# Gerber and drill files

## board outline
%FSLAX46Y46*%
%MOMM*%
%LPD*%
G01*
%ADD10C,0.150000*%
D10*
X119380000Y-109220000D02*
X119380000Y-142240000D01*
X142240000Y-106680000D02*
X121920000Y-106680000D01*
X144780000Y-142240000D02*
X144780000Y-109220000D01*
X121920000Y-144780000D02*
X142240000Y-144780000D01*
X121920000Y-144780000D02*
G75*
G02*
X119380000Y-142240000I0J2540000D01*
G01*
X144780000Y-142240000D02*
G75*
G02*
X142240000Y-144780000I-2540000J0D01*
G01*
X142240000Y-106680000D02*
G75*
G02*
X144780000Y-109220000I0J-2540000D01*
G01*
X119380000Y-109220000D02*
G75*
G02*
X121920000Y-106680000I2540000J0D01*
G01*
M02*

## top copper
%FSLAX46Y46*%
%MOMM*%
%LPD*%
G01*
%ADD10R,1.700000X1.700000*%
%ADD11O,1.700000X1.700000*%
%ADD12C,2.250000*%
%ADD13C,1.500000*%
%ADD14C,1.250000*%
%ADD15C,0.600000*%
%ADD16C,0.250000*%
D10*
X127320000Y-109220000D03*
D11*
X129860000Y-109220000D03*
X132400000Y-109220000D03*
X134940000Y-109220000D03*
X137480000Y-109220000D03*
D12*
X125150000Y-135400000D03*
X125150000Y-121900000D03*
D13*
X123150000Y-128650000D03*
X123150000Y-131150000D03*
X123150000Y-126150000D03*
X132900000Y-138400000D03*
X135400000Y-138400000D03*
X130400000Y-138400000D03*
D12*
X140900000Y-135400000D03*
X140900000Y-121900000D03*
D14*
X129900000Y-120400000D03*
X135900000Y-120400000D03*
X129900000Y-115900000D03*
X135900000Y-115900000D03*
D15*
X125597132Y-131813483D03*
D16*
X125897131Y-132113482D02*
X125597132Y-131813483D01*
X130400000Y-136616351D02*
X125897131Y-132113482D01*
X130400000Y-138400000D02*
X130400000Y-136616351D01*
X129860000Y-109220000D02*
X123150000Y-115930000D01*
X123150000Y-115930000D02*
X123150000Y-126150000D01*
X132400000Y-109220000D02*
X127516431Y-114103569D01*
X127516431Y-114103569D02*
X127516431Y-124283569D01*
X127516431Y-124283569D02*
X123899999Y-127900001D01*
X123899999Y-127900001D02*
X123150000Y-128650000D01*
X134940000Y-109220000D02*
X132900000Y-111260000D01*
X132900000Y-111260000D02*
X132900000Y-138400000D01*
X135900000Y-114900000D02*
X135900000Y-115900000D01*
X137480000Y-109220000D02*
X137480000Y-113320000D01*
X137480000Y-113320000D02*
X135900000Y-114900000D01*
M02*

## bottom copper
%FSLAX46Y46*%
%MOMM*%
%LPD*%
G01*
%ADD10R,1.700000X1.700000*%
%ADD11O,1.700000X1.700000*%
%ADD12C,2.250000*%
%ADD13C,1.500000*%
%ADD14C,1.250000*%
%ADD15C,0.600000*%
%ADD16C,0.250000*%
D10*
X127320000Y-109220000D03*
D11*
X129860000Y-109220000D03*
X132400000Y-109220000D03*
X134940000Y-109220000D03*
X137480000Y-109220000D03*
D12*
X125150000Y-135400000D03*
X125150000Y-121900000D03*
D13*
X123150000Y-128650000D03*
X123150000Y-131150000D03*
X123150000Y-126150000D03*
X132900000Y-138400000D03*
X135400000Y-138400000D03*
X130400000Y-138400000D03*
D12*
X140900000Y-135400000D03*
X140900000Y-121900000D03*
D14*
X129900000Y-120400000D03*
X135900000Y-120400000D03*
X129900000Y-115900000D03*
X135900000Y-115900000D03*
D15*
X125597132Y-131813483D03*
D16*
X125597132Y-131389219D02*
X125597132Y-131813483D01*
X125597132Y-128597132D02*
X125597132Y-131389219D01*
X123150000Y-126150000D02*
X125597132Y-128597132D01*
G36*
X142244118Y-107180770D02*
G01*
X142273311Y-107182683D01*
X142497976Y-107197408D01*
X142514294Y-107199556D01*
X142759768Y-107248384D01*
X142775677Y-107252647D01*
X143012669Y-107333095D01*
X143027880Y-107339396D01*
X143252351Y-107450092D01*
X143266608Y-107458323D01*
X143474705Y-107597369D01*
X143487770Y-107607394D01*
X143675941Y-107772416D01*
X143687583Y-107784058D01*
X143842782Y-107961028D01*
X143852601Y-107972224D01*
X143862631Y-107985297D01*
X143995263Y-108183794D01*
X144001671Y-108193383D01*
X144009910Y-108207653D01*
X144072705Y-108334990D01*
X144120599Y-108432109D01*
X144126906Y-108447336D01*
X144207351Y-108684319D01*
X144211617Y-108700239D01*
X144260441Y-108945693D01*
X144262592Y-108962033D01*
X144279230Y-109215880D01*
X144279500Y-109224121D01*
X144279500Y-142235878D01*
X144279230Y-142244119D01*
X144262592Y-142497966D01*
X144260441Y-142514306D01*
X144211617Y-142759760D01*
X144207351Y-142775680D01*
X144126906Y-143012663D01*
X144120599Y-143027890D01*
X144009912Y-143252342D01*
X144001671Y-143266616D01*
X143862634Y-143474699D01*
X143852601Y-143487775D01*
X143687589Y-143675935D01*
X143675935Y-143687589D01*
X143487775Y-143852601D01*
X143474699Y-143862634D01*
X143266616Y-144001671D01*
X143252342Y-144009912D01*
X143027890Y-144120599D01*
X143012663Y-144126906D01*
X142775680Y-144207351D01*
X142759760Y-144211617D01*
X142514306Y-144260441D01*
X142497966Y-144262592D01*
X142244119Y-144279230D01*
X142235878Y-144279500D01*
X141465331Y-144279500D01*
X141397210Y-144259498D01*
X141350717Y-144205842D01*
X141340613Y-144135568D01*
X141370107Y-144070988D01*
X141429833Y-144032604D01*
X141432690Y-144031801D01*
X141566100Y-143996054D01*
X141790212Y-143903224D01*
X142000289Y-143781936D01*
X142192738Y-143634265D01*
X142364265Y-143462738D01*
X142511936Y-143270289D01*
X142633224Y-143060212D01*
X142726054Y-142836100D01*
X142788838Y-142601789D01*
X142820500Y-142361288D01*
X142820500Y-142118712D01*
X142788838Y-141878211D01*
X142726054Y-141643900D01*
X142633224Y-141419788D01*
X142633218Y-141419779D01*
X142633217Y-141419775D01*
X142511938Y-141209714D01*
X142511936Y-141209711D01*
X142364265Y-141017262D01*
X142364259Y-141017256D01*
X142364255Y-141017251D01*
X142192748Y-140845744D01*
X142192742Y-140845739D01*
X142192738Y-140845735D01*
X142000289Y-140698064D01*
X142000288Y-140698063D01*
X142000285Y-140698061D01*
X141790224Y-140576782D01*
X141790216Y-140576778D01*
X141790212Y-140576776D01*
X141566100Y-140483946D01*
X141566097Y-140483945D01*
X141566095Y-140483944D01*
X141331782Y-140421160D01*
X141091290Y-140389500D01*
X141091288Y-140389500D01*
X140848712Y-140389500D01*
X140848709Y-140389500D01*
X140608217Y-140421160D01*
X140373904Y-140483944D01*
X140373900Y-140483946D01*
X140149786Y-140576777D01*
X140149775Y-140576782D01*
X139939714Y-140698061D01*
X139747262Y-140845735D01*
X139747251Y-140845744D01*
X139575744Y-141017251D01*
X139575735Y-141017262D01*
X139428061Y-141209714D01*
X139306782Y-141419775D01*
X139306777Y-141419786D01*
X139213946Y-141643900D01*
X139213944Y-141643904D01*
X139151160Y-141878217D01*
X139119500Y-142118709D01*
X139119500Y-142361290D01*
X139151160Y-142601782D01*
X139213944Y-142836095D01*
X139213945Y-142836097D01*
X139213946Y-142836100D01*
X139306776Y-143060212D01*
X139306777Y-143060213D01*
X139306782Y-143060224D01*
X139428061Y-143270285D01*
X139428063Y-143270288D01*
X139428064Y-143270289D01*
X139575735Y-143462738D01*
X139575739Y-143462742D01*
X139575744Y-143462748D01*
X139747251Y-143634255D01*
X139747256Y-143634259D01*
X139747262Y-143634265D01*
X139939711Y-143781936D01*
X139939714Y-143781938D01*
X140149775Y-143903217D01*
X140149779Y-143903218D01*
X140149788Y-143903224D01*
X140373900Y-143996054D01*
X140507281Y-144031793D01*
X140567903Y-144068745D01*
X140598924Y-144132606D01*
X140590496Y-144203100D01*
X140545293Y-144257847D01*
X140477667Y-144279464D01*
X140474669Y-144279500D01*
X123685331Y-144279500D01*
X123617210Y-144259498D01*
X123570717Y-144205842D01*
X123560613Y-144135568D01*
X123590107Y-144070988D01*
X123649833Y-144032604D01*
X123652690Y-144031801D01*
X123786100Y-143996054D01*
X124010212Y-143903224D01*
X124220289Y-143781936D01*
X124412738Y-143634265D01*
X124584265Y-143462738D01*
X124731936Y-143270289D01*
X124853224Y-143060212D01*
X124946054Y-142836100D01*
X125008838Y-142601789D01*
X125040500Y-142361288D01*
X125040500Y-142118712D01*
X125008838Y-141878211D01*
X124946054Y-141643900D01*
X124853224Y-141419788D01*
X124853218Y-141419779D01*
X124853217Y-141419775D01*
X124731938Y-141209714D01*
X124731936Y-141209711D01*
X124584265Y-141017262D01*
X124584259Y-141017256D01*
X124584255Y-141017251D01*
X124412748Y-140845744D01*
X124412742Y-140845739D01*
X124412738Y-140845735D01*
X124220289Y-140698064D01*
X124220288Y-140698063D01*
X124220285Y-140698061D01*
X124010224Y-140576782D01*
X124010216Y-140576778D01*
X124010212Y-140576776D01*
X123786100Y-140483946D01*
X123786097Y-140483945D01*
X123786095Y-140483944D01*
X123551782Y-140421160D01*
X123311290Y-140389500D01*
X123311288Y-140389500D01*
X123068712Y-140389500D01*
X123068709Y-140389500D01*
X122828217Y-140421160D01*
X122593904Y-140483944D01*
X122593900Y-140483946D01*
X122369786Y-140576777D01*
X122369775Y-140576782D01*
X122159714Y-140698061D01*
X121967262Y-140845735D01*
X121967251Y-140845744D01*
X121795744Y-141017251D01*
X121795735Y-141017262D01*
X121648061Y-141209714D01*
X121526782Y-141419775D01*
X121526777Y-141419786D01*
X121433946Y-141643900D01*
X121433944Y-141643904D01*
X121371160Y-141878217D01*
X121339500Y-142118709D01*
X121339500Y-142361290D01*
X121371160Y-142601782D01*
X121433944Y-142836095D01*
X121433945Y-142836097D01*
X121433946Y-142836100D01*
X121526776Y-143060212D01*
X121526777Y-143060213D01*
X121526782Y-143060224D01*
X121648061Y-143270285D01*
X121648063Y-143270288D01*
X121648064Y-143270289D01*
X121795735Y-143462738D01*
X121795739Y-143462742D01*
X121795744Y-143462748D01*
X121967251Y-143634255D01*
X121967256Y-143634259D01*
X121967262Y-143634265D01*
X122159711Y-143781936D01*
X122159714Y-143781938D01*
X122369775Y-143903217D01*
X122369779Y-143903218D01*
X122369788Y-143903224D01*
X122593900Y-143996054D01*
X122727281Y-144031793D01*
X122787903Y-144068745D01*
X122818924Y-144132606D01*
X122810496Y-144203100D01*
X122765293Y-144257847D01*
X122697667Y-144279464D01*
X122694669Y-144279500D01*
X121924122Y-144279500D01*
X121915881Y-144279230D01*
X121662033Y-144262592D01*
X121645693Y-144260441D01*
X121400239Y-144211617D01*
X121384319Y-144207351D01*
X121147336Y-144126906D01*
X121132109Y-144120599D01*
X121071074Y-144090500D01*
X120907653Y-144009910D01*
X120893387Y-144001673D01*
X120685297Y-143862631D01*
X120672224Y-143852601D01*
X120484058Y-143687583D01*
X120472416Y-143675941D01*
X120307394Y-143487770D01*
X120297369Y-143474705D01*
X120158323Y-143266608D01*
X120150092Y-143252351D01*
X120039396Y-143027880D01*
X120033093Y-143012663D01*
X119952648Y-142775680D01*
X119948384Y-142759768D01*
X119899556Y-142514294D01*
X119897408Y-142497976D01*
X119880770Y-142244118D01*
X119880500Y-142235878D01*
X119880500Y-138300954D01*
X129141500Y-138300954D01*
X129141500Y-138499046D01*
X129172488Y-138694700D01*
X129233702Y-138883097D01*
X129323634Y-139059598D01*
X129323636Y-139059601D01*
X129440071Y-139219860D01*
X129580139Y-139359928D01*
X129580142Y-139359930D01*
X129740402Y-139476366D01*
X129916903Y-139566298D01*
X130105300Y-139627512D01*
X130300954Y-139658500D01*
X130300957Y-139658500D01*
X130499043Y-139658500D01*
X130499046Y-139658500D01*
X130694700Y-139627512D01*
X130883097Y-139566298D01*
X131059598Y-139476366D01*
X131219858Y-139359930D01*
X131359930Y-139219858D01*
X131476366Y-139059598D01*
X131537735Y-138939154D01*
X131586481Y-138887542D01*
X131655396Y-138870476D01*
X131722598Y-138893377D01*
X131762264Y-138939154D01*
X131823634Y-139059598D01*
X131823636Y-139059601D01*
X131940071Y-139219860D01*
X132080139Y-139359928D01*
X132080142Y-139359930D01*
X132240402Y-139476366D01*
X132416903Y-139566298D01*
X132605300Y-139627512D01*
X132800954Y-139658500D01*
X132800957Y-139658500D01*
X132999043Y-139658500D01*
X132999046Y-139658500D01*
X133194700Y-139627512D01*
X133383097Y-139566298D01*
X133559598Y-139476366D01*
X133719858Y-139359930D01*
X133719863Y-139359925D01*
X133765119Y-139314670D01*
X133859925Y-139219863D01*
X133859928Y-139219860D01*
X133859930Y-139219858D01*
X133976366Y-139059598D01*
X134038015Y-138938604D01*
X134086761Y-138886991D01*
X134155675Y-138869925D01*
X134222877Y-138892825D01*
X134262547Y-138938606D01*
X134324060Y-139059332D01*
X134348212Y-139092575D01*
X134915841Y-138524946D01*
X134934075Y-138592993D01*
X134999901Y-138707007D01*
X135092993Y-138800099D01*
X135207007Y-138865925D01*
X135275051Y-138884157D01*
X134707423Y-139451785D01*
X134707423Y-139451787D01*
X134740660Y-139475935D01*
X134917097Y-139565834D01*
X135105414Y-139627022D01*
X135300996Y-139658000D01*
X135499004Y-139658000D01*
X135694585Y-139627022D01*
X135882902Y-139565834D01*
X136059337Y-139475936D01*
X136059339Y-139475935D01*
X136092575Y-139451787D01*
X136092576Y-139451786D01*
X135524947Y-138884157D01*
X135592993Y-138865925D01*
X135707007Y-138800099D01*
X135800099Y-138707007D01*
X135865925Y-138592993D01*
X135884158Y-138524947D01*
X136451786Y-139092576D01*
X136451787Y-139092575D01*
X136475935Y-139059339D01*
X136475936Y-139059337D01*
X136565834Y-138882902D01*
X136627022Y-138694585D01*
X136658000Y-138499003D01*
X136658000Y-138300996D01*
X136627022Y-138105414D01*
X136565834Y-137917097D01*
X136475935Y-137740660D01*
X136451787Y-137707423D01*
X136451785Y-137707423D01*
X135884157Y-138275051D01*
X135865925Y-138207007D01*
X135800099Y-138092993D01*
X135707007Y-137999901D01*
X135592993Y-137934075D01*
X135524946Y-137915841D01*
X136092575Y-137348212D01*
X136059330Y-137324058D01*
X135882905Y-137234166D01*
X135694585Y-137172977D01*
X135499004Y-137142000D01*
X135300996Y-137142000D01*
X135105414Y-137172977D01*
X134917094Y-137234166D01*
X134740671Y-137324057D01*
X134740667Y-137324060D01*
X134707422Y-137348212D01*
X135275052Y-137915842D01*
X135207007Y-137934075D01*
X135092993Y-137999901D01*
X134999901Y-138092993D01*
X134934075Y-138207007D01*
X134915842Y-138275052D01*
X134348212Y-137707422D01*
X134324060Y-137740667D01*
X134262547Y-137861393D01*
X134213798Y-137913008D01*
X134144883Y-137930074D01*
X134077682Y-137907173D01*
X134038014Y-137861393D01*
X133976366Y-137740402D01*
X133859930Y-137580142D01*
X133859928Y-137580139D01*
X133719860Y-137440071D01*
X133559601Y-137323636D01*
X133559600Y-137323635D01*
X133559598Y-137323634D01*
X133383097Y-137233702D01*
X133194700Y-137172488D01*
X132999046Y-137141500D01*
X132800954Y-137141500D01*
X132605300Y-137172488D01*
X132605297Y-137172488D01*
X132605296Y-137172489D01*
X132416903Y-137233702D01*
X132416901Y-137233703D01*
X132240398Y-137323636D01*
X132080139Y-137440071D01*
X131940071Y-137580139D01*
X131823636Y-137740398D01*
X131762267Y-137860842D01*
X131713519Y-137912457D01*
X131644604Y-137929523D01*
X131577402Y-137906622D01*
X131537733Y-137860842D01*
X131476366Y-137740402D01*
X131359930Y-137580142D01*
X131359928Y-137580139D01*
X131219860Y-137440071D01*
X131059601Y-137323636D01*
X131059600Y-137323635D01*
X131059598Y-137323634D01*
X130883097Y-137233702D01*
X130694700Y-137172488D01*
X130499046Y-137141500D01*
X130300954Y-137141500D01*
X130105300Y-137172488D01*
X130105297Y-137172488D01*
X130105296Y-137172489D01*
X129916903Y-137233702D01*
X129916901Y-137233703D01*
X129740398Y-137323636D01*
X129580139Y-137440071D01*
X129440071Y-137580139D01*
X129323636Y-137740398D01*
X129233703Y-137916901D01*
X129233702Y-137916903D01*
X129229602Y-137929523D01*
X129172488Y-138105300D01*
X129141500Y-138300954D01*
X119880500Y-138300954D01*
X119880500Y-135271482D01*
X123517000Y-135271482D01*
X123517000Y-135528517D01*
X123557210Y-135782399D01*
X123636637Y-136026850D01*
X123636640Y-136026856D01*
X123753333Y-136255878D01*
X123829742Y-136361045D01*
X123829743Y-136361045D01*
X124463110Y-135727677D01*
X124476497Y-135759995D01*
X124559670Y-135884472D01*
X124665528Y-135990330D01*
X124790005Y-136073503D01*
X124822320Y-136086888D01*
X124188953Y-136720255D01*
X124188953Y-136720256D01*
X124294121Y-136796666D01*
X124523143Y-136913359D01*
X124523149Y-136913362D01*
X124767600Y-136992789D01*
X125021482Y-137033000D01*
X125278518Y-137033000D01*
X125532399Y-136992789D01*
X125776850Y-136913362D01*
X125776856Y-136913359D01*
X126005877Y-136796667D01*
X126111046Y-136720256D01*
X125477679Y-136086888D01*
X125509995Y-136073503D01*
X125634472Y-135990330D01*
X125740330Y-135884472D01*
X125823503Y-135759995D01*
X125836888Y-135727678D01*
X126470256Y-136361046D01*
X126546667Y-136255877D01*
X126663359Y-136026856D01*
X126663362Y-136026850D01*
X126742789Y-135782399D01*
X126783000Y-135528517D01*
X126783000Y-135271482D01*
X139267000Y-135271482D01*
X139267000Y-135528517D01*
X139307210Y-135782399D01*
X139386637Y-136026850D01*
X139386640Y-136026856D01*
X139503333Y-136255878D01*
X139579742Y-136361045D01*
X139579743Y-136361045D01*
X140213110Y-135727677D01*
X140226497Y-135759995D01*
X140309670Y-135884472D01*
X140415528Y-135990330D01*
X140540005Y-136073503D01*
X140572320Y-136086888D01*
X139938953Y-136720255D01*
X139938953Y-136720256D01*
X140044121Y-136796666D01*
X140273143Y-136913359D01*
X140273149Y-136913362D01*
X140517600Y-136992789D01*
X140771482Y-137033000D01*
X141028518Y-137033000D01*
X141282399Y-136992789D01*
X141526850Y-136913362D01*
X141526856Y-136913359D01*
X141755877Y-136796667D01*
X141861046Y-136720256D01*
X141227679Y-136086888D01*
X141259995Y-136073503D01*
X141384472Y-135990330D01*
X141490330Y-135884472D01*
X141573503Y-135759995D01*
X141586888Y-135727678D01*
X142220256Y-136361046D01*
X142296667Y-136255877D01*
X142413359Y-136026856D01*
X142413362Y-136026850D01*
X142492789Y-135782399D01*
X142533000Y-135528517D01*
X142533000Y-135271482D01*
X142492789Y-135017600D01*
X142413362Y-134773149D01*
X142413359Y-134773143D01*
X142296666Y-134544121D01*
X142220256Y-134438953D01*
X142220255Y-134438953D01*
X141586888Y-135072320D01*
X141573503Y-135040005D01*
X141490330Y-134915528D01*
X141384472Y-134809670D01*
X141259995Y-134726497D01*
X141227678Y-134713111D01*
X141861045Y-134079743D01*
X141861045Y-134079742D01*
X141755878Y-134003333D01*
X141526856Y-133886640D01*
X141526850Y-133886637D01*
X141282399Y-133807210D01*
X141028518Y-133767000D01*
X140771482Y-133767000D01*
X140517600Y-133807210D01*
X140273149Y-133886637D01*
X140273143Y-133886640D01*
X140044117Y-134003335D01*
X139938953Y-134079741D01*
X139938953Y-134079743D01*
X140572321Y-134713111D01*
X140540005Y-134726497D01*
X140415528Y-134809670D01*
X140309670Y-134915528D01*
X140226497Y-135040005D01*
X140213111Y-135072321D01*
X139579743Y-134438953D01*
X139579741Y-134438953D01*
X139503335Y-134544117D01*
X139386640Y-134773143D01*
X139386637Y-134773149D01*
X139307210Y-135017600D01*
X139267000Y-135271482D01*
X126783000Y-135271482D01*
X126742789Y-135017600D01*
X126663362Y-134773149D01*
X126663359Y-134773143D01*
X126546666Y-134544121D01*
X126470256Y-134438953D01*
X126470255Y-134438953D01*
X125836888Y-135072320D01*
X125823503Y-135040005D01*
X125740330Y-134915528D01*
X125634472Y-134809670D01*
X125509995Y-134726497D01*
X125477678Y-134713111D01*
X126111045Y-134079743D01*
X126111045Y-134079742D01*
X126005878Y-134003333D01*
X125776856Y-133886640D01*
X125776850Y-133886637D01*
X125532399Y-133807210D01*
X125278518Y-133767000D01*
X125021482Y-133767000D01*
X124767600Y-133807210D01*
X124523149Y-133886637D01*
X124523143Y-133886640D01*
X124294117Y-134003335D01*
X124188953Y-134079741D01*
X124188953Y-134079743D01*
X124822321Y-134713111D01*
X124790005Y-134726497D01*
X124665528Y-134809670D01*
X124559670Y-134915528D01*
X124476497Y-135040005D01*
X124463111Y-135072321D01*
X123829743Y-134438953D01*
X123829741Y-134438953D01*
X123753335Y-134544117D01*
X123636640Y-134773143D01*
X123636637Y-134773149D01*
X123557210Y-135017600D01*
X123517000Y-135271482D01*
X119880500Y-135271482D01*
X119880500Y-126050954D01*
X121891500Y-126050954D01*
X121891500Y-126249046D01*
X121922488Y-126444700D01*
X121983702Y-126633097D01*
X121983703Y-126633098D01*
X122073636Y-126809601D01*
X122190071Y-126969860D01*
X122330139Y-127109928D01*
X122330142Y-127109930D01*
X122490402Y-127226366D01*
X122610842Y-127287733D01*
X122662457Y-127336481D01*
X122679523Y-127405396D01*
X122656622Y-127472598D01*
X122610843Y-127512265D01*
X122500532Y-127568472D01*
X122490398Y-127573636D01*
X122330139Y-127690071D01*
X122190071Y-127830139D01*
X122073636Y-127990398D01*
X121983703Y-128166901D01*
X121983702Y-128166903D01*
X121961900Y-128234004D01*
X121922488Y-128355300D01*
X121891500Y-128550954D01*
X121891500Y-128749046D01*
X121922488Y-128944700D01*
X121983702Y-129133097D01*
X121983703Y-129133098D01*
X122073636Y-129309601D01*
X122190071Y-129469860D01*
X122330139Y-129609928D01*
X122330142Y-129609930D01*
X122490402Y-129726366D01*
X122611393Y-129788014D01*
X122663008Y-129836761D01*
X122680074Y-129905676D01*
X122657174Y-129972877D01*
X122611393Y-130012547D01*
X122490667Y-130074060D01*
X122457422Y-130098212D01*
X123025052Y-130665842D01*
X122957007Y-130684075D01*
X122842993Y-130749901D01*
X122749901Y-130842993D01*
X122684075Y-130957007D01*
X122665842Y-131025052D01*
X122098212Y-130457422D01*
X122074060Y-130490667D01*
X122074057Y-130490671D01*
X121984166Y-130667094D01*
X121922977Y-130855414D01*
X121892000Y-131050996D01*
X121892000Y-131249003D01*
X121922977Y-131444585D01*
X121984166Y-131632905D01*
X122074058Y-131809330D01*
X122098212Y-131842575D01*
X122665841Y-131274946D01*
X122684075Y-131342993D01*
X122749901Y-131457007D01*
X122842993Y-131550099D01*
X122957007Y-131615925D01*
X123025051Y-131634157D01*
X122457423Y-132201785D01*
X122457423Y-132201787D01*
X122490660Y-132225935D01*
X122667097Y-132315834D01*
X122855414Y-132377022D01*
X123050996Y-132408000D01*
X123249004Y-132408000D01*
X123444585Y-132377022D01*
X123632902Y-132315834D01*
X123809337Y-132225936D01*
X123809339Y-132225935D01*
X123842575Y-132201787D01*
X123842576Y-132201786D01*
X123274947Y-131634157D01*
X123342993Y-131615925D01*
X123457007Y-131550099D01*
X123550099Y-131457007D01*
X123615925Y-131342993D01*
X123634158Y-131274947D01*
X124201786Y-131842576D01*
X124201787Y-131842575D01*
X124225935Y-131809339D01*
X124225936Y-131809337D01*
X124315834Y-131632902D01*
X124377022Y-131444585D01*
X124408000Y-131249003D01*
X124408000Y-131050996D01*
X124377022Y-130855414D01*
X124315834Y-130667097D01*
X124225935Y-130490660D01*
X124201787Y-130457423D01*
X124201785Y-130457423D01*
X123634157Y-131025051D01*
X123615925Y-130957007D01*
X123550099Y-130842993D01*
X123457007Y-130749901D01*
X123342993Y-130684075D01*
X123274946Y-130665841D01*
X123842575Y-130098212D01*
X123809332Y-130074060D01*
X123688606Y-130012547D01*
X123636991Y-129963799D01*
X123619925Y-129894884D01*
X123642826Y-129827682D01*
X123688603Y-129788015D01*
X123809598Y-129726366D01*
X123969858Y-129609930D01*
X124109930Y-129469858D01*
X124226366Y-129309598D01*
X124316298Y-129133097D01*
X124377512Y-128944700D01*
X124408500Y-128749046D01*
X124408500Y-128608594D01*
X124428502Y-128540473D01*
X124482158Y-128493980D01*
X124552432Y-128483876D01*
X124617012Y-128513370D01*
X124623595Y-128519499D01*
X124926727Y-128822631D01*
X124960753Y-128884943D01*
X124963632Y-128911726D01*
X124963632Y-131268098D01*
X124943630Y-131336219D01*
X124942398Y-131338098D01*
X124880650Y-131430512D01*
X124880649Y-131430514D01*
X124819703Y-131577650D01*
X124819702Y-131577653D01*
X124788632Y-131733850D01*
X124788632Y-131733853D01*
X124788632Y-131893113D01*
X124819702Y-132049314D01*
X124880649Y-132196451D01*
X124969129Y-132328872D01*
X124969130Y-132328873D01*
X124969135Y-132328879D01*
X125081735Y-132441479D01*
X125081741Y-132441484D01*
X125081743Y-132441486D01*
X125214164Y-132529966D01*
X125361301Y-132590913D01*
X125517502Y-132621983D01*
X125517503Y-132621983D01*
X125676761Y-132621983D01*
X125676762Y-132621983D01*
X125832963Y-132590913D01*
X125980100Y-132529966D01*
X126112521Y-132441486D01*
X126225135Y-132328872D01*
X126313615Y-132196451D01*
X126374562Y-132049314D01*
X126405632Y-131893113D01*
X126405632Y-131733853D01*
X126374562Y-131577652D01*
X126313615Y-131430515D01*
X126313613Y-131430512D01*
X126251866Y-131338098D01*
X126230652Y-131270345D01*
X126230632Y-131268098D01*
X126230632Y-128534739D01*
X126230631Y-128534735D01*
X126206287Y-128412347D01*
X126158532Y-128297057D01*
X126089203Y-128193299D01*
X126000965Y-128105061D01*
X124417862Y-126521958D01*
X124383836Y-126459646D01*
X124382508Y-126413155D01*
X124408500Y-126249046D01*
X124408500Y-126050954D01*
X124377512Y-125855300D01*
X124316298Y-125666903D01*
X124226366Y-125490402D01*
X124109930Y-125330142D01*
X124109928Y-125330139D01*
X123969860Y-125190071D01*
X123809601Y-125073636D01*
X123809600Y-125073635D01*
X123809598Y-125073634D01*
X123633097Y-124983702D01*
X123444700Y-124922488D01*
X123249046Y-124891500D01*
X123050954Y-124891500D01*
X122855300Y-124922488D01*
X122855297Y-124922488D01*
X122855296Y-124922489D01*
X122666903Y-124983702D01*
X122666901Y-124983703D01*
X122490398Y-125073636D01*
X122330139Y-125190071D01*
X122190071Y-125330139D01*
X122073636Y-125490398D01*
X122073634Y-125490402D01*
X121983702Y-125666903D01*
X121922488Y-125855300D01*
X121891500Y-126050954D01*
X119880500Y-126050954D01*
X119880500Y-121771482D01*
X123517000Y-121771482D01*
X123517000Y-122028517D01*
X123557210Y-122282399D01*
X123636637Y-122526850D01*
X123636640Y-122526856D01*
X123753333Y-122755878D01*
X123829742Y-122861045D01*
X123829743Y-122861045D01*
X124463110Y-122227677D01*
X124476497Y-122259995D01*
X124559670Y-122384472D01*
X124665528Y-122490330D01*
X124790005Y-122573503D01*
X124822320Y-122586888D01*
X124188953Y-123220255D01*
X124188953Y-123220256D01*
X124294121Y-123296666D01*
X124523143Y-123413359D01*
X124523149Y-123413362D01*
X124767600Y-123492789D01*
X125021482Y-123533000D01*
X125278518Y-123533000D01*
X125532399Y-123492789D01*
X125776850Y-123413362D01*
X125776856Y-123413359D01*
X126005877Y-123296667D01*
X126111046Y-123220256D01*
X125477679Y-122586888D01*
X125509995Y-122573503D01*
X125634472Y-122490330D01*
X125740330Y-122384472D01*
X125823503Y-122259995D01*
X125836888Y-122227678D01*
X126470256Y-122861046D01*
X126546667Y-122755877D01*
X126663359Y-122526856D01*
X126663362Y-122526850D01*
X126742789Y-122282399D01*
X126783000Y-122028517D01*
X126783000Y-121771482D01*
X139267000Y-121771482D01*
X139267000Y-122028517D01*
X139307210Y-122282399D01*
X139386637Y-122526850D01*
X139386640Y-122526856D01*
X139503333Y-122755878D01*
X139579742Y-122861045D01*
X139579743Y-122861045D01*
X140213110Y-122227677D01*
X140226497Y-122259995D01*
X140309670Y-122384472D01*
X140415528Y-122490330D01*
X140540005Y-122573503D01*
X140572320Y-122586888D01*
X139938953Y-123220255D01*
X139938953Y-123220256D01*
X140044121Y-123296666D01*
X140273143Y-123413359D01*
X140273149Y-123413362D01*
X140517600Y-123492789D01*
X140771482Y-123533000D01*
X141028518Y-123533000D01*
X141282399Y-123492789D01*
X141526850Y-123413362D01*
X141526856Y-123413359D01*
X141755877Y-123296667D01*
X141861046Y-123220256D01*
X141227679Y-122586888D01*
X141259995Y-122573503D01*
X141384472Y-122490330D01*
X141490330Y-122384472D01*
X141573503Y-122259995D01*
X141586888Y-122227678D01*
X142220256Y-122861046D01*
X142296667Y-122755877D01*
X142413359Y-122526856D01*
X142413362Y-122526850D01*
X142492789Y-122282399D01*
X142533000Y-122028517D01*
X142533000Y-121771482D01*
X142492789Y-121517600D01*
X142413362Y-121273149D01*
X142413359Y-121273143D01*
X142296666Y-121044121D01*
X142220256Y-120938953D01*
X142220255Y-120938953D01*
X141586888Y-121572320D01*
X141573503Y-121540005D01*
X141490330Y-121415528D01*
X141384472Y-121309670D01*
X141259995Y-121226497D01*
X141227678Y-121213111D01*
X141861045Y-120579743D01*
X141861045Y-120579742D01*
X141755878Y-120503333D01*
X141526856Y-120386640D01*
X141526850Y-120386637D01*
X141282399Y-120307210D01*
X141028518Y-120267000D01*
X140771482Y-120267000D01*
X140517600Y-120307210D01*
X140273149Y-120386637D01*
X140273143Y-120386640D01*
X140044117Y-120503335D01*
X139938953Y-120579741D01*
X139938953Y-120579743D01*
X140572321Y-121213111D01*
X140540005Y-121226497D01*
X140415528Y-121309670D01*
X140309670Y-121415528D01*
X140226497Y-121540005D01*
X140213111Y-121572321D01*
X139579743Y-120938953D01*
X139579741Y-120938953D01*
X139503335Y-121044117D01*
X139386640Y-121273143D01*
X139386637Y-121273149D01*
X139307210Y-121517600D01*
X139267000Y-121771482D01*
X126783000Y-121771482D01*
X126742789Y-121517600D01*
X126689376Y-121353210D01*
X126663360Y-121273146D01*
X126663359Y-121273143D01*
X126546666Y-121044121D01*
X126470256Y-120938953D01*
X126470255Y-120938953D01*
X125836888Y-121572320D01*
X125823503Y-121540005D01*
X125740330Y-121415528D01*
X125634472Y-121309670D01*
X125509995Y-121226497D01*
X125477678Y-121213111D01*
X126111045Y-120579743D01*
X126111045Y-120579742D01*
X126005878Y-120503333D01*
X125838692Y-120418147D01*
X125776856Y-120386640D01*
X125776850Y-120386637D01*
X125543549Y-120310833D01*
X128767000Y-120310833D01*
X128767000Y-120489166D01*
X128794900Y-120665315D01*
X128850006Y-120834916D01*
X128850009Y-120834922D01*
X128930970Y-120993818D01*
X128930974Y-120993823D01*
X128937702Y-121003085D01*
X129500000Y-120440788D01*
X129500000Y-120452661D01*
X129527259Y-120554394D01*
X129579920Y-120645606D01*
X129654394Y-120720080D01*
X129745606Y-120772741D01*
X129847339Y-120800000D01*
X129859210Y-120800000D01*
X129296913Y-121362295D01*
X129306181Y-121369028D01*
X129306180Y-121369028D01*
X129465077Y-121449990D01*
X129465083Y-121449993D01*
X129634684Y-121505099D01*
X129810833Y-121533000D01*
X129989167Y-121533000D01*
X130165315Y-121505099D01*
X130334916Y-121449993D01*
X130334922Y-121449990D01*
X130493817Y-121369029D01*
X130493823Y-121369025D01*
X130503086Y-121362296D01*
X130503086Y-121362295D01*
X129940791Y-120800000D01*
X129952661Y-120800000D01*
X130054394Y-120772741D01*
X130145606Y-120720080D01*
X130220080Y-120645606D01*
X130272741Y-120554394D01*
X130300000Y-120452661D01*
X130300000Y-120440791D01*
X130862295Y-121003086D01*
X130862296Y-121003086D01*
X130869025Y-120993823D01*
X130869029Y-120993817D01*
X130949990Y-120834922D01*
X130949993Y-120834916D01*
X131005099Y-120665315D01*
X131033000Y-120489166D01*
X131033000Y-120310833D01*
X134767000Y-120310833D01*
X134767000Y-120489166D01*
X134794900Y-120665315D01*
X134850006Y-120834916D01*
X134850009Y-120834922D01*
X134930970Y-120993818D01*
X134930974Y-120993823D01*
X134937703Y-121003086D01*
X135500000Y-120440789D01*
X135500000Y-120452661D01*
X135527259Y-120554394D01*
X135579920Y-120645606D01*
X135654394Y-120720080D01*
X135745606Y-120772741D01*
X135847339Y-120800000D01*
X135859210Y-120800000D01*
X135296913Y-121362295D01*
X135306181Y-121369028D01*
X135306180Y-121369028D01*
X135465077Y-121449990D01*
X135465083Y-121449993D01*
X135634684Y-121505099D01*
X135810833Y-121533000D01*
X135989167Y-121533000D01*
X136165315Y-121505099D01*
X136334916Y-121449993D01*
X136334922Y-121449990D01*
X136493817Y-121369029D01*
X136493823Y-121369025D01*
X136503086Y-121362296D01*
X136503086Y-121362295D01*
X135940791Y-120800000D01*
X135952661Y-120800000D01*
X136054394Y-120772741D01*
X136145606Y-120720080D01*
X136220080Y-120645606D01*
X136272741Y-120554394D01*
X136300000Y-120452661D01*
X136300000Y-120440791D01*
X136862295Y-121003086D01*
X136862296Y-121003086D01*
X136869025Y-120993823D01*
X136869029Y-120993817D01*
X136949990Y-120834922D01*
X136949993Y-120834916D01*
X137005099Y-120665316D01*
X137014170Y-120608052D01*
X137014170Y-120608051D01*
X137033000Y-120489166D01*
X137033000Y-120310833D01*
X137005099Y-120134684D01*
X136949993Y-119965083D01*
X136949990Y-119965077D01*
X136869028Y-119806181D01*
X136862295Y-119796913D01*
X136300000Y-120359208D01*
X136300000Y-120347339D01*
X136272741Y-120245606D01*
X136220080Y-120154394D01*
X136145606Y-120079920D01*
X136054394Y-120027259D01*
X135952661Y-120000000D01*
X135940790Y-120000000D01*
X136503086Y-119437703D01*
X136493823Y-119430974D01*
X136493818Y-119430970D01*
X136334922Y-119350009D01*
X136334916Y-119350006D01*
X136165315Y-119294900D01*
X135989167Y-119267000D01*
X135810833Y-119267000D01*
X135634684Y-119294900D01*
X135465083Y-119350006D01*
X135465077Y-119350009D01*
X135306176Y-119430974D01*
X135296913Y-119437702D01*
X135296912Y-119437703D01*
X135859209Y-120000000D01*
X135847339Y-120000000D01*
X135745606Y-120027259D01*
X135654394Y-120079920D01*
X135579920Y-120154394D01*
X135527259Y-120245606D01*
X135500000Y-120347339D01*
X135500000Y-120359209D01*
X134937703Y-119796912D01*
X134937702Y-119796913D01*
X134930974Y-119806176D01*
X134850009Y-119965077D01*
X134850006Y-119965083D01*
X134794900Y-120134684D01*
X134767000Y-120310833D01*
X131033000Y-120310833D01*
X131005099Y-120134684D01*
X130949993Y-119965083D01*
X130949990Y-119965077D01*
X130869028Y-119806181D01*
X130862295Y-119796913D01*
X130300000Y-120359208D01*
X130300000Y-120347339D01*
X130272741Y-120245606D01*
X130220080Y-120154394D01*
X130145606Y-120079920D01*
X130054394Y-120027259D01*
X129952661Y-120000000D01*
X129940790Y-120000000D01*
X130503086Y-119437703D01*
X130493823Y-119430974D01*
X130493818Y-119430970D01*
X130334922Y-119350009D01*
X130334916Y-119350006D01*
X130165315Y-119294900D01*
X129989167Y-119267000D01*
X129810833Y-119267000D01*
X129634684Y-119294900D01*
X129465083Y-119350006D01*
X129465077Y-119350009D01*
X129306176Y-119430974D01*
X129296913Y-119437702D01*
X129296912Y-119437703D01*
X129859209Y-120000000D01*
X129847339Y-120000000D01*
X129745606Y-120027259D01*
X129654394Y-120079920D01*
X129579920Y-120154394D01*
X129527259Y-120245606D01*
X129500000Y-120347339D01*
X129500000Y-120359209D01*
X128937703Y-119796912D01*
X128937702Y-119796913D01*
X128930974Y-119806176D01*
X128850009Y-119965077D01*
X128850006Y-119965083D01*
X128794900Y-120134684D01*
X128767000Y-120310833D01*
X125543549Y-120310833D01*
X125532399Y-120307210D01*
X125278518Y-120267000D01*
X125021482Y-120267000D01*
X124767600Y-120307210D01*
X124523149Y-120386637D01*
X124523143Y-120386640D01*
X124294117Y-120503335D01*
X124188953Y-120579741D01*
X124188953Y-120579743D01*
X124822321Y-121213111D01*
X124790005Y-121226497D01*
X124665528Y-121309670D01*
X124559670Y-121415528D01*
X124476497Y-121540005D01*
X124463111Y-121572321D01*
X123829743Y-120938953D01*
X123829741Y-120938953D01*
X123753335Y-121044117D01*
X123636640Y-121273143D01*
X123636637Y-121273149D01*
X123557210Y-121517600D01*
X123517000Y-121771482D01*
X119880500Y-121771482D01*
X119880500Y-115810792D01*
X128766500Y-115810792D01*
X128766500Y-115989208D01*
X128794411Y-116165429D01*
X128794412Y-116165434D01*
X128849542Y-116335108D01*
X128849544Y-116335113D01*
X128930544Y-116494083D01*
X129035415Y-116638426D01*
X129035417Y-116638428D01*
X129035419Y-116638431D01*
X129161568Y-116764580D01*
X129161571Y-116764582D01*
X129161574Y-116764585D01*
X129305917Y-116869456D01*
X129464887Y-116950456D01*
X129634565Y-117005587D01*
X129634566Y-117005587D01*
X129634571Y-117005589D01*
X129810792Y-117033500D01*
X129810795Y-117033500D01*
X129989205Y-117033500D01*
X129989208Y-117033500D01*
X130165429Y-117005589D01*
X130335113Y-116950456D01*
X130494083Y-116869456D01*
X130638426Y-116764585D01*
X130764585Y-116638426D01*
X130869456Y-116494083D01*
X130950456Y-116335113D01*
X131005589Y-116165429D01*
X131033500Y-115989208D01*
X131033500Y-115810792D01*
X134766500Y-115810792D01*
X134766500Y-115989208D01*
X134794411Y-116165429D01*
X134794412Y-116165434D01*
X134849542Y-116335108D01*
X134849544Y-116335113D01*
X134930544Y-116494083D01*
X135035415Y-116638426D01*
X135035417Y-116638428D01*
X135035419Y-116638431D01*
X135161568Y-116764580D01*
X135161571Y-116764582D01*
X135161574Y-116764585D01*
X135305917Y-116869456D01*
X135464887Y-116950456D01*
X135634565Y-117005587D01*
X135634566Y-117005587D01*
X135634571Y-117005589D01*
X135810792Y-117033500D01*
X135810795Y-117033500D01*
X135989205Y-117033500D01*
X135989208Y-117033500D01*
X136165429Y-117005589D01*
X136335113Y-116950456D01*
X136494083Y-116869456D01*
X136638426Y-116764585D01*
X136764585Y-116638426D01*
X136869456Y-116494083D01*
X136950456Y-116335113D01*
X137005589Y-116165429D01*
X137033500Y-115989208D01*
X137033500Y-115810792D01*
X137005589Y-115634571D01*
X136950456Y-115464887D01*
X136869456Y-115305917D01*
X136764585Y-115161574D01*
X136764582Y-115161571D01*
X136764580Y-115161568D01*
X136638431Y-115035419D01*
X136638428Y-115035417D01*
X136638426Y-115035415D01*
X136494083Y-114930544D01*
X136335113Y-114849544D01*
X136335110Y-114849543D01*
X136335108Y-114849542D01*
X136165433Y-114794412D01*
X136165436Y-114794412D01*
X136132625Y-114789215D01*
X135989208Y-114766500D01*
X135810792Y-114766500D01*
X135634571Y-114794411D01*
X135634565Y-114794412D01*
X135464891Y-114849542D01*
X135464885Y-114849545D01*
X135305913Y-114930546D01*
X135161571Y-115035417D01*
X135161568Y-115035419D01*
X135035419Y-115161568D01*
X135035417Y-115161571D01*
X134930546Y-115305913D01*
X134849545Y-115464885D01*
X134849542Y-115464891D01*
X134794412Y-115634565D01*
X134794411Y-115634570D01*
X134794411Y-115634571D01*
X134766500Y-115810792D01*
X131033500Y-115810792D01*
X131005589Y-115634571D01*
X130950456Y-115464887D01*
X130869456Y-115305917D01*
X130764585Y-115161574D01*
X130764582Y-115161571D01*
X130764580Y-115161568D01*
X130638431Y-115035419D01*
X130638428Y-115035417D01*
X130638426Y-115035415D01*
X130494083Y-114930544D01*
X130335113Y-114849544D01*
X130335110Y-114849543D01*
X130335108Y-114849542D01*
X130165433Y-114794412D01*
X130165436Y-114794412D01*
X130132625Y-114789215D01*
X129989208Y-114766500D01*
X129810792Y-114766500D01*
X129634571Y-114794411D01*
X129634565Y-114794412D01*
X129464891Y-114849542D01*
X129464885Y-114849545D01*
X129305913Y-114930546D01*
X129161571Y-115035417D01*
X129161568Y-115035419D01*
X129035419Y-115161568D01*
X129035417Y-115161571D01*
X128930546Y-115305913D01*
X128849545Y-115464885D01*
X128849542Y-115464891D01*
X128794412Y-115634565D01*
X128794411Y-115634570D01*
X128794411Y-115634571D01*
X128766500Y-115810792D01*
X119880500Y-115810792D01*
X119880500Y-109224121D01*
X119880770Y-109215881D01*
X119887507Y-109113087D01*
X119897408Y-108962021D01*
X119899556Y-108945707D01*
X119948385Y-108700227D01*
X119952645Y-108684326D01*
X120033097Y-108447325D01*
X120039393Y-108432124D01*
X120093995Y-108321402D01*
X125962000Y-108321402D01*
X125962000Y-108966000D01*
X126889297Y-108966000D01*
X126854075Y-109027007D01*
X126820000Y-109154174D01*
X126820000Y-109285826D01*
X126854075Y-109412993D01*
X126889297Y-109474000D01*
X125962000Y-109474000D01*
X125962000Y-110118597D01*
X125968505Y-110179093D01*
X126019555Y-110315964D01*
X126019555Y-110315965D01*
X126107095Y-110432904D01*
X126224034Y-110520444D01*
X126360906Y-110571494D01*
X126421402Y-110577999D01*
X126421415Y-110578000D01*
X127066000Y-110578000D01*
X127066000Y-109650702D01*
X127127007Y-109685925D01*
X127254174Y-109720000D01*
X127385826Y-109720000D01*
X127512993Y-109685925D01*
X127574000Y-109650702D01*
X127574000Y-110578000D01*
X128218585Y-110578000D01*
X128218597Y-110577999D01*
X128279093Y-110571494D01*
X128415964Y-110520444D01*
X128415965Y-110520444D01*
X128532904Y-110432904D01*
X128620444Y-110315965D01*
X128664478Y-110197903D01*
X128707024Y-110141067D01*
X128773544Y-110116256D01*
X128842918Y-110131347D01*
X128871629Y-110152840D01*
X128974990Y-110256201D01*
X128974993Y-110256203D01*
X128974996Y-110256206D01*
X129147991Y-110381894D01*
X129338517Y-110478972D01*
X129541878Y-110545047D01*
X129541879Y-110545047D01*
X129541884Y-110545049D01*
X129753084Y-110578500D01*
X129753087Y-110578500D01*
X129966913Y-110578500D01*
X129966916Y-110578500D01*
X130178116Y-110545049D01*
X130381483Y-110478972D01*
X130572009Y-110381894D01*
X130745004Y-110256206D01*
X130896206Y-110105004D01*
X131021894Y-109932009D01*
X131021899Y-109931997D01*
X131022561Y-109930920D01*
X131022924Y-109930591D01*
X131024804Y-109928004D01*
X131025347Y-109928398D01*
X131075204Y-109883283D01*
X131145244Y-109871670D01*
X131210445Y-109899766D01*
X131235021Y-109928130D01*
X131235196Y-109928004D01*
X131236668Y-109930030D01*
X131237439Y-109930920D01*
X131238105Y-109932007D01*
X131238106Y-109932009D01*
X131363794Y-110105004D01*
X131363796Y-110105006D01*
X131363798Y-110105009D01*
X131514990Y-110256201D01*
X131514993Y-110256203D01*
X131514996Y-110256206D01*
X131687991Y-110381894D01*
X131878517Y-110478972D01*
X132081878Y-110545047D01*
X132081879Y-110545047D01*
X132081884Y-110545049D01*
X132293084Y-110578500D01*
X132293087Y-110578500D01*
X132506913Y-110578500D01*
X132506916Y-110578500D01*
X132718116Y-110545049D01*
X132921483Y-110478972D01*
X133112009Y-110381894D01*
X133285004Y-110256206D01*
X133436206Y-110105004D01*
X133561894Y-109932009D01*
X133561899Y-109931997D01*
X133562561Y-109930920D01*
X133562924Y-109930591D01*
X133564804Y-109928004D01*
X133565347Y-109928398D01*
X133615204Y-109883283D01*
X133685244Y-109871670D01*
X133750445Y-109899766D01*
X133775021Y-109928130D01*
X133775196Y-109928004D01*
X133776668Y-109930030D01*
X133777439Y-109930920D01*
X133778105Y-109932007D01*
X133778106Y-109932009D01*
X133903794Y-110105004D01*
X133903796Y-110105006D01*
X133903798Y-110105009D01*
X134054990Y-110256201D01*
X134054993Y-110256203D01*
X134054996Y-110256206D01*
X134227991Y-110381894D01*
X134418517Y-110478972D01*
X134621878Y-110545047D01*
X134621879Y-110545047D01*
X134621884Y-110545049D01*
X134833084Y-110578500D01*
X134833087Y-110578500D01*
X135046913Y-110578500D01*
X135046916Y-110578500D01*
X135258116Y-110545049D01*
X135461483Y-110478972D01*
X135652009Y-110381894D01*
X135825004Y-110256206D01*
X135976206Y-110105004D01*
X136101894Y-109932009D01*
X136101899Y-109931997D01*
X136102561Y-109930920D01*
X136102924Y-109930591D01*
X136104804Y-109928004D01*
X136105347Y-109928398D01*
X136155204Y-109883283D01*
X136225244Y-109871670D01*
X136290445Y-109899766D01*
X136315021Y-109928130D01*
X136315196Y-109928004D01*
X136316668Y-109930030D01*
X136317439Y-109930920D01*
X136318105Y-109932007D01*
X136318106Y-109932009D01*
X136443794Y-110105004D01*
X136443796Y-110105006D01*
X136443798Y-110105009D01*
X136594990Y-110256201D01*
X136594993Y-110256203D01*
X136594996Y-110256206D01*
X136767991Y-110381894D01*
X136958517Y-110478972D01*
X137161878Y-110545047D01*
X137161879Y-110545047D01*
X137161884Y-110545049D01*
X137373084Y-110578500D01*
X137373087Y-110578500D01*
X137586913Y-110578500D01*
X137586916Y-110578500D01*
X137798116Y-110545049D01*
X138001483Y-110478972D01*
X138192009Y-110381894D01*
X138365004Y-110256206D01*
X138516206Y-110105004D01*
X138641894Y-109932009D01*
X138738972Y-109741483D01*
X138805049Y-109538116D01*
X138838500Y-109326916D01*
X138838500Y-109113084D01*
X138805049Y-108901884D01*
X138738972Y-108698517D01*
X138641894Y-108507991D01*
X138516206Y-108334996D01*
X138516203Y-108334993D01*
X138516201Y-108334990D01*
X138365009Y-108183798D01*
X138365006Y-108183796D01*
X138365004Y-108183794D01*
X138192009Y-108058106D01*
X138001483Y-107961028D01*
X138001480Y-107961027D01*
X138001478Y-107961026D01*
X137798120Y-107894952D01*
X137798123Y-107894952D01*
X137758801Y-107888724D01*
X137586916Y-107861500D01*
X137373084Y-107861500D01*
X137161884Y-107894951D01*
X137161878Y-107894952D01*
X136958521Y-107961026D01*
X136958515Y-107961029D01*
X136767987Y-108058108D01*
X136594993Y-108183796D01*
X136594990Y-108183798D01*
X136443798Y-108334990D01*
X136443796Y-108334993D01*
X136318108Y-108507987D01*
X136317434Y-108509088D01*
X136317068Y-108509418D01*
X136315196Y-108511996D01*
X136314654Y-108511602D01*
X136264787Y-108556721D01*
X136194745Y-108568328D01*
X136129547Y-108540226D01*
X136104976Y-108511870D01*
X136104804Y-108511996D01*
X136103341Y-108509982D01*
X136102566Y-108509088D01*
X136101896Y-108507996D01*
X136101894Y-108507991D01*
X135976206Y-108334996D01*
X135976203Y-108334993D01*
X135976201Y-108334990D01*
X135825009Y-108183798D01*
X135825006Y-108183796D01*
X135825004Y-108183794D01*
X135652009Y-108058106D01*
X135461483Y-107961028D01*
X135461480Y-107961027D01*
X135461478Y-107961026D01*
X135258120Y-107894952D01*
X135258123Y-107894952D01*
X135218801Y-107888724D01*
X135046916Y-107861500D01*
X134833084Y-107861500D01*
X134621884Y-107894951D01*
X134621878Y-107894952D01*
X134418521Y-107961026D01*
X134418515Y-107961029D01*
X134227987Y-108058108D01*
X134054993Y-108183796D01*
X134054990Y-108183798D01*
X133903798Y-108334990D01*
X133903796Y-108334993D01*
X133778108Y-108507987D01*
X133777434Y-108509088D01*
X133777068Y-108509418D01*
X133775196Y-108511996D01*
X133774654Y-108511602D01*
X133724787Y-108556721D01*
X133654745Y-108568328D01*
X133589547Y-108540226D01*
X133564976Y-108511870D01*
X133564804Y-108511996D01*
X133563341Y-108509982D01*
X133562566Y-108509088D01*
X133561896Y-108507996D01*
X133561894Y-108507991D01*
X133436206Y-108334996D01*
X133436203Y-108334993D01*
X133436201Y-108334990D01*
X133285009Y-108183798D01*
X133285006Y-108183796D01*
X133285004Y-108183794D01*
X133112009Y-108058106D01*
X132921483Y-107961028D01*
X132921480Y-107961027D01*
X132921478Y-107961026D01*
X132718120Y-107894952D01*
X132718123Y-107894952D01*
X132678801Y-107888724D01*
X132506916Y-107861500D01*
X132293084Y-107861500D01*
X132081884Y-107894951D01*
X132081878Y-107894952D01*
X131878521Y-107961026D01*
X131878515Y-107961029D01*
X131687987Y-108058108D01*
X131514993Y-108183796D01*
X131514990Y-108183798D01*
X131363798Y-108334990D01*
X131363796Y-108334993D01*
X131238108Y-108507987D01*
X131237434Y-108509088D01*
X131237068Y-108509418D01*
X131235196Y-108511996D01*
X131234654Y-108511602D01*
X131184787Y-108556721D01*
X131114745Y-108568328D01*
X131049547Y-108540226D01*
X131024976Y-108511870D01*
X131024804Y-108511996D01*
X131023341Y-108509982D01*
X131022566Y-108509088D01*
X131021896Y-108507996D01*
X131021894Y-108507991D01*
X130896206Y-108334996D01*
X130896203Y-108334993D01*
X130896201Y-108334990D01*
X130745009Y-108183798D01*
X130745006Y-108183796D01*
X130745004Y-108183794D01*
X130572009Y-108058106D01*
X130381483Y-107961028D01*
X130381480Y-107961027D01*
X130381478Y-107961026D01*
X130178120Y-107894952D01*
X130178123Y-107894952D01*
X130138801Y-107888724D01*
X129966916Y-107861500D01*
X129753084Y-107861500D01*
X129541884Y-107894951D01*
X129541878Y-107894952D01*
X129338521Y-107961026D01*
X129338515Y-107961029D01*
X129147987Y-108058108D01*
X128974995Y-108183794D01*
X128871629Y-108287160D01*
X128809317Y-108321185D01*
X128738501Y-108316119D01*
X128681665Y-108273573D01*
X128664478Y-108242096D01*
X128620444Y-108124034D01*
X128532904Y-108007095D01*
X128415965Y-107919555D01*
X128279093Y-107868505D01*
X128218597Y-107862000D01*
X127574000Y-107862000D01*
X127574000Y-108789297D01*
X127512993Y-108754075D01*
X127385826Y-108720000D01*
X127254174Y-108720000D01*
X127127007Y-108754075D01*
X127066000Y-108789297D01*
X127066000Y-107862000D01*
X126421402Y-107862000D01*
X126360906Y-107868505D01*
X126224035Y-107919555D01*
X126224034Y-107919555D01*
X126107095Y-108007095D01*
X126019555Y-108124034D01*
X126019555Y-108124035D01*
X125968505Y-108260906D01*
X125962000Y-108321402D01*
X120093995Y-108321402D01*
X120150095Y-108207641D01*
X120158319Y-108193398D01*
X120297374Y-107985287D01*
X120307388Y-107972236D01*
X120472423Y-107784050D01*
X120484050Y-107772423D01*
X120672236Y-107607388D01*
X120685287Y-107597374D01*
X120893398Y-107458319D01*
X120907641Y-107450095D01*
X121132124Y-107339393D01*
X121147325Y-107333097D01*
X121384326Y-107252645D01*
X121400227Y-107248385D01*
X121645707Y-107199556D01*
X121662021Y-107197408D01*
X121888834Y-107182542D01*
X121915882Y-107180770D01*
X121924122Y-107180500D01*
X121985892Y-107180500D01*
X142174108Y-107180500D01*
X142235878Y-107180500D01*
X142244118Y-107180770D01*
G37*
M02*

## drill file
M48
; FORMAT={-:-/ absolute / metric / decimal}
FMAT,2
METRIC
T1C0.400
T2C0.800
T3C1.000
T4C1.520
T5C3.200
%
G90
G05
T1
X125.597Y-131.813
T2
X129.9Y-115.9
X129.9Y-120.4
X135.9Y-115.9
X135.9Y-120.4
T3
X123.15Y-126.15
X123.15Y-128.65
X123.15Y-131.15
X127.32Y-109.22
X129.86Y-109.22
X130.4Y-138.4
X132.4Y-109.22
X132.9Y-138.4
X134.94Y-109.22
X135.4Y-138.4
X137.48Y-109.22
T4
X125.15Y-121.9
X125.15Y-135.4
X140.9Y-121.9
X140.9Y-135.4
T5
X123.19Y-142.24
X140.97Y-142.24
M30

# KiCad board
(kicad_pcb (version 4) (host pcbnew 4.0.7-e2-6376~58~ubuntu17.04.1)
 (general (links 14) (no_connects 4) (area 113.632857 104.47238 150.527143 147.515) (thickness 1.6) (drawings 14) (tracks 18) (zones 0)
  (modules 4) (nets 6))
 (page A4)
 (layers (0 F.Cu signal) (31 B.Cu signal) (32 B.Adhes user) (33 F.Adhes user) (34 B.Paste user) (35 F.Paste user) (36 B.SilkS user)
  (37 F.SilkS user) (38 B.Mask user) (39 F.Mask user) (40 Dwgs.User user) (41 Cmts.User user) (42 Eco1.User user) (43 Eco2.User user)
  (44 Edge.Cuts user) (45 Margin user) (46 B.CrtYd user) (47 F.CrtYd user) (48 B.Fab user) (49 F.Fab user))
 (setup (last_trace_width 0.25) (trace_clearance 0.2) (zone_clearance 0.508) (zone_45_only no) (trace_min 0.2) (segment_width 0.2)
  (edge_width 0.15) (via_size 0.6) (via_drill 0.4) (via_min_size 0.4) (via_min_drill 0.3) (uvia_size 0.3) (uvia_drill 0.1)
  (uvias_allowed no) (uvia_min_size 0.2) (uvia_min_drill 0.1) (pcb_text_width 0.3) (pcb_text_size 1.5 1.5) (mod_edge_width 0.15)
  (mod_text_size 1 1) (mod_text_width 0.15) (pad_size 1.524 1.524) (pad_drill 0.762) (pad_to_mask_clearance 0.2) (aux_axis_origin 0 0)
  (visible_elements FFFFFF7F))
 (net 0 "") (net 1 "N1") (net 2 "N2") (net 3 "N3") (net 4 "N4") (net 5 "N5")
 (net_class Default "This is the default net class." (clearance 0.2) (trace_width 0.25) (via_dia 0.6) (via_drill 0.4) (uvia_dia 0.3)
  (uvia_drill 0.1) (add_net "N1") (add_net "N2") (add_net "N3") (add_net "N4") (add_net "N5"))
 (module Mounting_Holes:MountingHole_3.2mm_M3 (layer F.Cu) (at 123.19 142.24)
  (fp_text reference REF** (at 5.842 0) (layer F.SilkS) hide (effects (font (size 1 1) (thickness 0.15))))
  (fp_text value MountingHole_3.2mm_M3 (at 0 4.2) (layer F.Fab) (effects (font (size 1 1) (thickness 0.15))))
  (pad 1 np_thru_hole circle (at 0 0) (size 3.2 3.2) (drill 3.2) (layers *.Cu *.Mask)))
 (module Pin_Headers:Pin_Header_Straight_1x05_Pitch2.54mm (layer F.Cu) (at 127.32 109.22 90)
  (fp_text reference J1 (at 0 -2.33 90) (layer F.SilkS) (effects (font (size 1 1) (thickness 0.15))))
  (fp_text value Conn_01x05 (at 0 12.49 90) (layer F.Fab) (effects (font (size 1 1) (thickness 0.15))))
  (pad 1 thru_hole rect (at 0 0 90) (size 1.7 1.7) (drill 1) (layers *.Cu *.Mask) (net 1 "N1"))
  (pad 2 thru_hole oval (at 0 2.54 90) (size 1.7 1.7) (drill 1) (layers *.Cu *.Mask) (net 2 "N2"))
  (pad 3 thru_hole oval (at 0 5.08 90) (size 1.7 1.7) (drill 1) (layers *.Cu *.Mask) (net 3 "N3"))
  (pad 4 thru_hole oval (at 0 7.62 90) (size 1.7 1.7) (drill 1) (layers *.Cu *.Mask) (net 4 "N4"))
  (pad 5 thru_hole oval (at 0 10.16 90) (size 1.7 1.7) (drill 1) (layers *.Cu *.Mask) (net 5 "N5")))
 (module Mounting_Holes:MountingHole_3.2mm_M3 (layer F.Cu) (at 140.97 142.24)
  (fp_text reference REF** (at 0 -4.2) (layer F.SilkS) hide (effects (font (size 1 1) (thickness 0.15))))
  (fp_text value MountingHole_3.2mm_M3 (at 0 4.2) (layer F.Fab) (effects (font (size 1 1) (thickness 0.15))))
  (pad 1 np_thru_hole circle (at 0 0) (size 3.2 3.2) (drill 3.2) (layers *.Cu *.Mask)))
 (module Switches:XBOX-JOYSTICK (layer F.Cu) (at 132.9 128.9 90)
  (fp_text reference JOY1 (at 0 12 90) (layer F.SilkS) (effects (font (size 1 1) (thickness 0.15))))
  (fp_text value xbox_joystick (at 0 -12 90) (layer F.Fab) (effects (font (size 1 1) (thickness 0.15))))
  (pad 1 thru_hole circle (at -6.5 -7.75 90) (size 2.25 2.25) (drill 1.52) (layers *.Cu *.Mask) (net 1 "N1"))
  (pad 1 thru_hole circle (at 7 -7.75 90) (size 2.25 2.25) (drill 1.52) (layers *.Cu *.Mask) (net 1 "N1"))
  (pad 3 thru_hole circle (at 0.25 -9.75 90) (size 1.5 1.5) (drill 1) (layers *.Cu *.Mask) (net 3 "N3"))
  (pad 2 thru_hole circle (at -2.25 -9.75 90) (size 1.5 1.5) (drill 1) (layers *.Cu *.Mask) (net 1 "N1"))
  (pad 4 thru_hole circle (at 2.75 -9.75 90) (size 1.5 1.5) (drill 1) (layers *.Cu *.Mask) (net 2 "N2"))
  (pad 6 thru_hole circle (at -9.5 0 180) (size 1.5 1.5) (drill 1) (layers *.Cu *.Mask) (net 4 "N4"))
  (pad 5 thru_hole circle (at -9.5 2.5 180) (size 1.5 1.5) (drill 1) (layers *.Cu *.Mask) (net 1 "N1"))
  (pad 7 thru_hole circle (at -9.5 -2.5 180) (size 1.5 1.5) (drill 1) (layers *.Cu *.Mask) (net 2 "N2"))
  (pad 1 thru_hole circle (at -6.5 8 90) (size 2.25 2.25) (drill 1.52) (layers *.Cu *.Mask) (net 1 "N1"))
  (pad 1 thru_hole circle (at 7 8 90) (size 2.25 2.25) (drill 1.52) (layers *.Cu *.Mask) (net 1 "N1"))
  (pad 8 thru_hole circle (at 8.5 -3 180) (size 1.25 1.25) (drill 0.8) (layers *.Cu *.Mask) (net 1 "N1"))
  (pad 8 thru_hole circle (at 8.5 3 180) (size 1.25 1.25) (drill 0.8) (layers *.Cu *.Mask) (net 1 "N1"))
  (pad 9 thru_hole circle (at 13 -3 180) (size 1.25 1.25) (drill 0.8) (layers *.Cu *.Mask) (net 5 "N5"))
  (pad 9 thru_hole circle (at 13 3 180) (size 1.25 1.25) (drill 0.8) (layers *.Cu *.Mask) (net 5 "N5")))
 (gr_line (start 119.38 109.22) (end 119.38 142.24) (layer Edge.Cuts) (width 0.15))
 (gr_line (start 142.24 106.68) (end 121.92 106.68) (layer Edge.Cuts) (width 0.15))
 (gr_line (start 144.78 142.24) (end 144.78 109.22) (layer Edge.Cuts) (width 0.15))
 (gr_line (start 121.92 144.78) (end 142.24 144.78) (layer Edge.Cuts) (width 0.15))
 (gr_arc (start 121.92 142.24) (end 121.92 144.78) (angle 90) (layer Edge.Cuts) (width 0.15))
 (gr_arc (start 142.24 142.24) (end 144.78 142.24) (angle 90) (layer Edge.Cuts) (width 0.15))
 (gr_arc (start 142.24 109.22) (end 142.24 106.68) (angle 90) (layer Edge.Cuts) (width 0.15))
 (gr_arc (start 121.92 109.22) (end 119.38 109.22) (angle 90) (layer Edge.Cuts) (width 0.15))
 (segment (start 125.597132 131.389219) (end 125.597132 131.813483) (width 0.25) (layer B.Cu) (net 2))
 (segment (start 125.597132 128.597132) (end 125.597132 131.389219) (width 0.25) (layer B.Cu) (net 2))
 (segment (start 123.15 126.15) (end 125.597132 128.597132) (width 0.25) (layer B.Cu) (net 2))
 (segment (start 125.897131 132.113482) (end 125.597132 131.813483) (width 0.25) (layer F.Cu) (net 2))
 (segment (start 130.4 136.616351) (end 125.897131 132.113482) (width 0.25) (layer F.Cu) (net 2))
 (segment (start 130.4 138.4) (end 130.4 136.616351) (width 0.25) (layer F.Cu) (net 2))
 (via (at 125.597132 131.813483) (size 0.6) (drill 0.4) (layers F.Cu B.Cu) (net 2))
 (segment (start 129.86 109.22) (end 123.15 115.93) (width 0.25) (layer F.Cu) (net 2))
 (segment (start 123.15 115.93) (end 123.15 126.15) (width 0.25) (layer F.Cu) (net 2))
 (segment (start 132.4 109.22) (end 127.516431 114.103569) (width 0.25) (layer F.Cu) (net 3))
 (segment (start 127.516431 114.103569) (end 127.516431 124.283569) (width 0.25) (layer F.Cu) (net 3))
 (segment (start 127.516431 124.283569) (end 123.899999 127.900001) (width 0.25) (layer F.Cu) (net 3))
 (segment (start 123.899999 127.900001) (end 123.15 128.65) (width 0.25) (layer F.Cu) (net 3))
 (segment (start 134.94 109.22) (end 132.9 111.26) (width 0.25) (layer F.Cu) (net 4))
 (segment (start 132.9 111.26) (end 132.9 138.4) (width 0.25) (layer F.Cu) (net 4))
 (segment (start 135.9 114.9) (end 135.9 115.9) (width 0.25) (layer F.Cu) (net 5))
 (segment (start 137.48 109.22) (end 137.48 113.32) (width 0.25) (layer F.Cu) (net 5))
 (segment (start 137.48 113.32) (end 135.9 114.9) (width 0.25) (layer F.Cu) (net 5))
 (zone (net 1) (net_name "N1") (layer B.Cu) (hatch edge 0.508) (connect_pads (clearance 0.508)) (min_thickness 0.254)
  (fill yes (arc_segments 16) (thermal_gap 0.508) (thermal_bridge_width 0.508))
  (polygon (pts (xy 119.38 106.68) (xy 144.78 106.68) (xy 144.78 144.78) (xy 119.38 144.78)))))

